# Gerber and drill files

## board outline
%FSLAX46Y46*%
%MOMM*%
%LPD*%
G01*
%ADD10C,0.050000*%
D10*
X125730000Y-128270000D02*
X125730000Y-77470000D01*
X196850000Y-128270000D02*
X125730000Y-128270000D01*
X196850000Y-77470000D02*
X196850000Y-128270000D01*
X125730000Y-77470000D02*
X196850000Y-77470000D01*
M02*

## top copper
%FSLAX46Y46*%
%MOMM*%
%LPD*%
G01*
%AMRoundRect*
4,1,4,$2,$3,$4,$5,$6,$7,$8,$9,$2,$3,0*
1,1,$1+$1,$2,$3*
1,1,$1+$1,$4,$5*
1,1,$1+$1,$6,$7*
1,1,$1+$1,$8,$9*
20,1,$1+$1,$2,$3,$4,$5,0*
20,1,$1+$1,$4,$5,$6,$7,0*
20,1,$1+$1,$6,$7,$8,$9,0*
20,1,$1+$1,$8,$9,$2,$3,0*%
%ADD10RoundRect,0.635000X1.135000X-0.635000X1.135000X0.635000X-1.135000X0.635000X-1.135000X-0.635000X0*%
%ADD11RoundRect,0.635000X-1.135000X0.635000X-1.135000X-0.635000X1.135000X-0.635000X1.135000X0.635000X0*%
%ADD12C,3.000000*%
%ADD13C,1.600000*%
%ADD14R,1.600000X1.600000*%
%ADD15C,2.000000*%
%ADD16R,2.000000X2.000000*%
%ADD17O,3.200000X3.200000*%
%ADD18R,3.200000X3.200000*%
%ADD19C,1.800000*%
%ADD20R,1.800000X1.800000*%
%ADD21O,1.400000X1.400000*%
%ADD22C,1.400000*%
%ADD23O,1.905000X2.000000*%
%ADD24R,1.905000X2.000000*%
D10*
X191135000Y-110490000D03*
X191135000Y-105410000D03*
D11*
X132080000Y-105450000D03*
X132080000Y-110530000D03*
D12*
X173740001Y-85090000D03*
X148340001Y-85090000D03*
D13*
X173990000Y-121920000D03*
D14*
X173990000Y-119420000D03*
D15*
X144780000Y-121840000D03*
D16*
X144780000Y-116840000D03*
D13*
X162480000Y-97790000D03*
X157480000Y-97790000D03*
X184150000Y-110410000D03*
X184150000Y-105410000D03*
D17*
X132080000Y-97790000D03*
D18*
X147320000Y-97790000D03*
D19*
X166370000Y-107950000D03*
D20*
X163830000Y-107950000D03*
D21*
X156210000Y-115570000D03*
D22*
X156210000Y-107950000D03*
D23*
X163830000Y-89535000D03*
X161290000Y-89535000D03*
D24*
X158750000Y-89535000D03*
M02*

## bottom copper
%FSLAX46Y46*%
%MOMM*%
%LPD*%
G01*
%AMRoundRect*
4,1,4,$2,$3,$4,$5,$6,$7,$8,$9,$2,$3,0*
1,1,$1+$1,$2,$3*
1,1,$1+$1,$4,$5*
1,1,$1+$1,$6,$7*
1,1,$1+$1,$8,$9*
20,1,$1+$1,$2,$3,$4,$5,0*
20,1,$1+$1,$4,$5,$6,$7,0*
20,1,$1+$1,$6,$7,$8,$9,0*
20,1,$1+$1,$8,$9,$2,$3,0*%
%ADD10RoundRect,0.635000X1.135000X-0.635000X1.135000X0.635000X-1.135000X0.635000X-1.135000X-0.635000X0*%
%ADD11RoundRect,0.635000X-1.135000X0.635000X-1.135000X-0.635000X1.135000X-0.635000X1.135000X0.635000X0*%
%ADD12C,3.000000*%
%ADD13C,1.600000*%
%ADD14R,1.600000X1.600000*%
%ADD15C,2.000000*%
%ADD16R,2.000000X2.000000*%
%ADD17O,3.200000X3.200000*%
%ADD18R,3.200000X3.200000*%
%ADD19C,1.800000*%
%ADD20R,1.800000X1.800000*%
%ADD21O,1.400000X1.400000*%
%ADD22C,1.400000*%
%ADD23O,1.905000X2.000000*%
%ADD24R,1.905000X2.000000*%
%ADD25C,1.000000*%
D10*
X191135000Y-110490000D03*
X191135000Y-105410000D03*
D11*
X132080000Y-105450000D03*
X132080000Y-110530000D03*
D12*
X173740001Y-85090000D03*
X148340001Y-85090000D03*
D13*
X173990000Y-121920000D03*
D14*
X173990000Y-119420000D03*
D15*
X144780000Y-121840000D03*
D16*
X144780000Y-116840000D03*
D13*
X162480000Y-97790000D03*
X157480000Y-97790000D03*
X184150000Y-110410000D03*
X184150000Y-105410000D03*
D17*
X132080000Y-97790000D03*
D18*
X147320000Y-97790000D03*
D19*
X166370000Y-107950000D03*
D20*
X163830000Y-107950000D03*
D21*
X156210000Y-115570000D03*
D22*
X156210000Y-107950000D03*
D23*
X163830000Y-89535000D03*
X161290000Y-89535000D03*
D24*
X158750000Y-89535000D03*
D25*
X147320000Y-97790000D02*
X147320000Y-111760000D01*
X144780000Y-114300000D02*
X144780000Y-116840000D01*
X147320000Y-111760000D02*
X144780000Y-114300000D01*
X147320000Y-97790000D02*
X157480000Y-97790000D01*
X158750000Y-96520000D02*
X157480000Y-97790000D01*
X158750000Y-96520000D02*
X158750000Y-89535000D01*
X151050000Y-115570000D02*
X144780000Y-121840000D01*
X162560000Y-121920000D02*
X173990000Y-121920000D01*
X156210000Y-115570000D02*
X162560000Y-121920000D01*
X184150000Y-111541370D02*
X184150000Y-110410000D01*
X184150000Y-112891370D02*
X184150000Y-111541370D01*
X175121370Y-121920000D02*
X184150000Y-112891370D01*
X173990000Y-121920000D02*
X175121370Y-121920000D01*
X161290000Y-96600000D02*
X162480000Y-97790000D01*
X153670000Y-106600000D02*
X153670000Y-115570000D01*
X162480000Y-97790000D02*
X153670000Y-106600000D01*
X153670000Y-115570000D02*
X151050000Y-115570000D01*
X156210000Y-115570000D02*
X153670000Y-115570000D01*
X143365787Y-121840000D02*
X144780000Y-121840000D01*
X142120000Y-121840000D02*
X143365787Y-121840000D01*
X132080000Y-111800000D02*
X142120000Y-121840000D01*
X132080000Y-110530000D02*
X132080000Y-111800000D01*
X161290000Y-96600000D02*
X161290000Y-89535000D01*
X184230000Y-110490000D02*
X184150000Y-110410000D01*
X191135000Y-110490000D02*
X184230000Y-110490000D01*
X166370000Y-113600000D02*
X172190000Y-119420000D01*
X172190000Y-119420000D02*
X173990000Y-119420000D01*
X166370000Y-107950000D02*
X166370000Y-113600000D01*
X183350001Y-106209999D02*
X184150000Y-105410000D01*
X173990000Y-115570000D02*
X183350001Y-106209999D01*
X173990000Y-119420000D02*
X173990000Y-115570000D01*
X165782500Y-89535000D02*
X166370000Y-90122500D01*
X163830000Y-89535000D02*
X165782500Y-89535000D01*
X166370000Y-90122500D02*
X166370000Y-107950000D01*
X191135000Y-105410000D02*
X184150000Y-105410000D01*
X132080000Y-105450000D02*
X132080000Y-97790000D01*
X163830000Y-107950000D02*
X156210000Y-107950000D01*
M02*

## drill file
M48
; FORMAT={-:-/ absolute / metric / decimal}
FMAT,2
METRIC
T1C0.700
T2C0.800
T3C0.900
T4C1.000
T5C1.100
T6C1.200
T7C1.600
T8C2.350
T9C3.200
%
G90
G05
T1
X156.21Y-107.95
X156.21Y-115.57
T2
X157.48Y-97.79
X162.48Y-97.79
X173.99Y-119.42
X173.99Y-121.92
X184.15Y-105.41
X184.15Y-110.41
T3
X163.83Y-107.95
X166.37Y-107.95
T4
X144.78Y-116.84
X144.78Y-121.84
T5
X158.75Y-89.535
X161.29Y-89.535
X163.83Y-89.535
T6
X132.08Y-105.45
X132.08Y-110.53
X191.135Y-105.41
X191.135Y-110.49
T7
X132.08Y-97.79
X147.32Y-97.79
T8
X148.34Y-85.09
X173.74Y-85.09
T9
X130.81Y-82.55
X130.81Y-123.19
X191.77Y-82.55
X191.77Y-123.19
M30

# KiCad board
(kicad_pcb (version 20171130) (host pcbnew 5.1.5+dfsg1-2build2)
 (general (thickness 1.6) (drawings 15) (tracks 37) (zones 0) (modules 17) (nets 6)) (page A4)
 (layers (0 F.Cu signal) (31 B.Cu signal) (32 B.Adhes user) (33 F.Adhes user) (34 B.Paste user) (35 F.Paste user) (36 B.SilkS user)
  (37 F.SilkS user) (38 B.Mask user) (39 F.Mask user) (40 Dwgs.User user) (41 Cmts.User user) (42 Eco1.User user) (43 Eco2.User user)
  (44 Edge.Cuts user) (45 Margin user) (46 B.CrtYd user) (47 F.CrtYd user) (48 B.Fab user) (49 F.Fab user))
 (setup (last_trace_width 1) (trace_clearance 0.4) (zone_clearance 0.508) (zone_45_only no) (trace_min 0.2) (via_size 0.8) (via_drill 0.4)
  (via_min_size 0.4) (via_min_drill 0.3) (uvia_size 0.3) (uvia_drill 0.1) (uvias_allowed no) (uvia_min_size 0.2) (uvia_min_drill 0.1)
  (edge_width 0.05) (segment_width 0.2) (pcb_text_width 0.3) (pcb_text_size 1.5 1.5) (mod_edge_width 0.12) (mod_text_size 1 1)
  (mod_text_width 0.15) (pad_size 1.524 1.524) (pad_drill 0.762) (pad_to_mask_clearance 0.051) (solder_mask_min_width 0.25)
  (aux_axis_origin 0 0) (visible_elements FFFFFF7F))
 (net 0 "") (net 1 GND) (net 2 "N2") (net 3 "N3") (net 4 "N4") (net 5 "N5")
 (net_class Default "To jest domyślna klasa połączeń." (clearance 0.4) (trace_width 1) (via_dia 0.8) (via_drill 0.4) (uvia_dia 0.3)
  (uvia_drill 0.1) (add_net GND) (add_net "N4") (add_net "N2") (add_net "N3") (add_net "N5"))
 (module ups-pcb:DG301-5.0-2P (layer F.Cu) (at 191.135 107.99 90)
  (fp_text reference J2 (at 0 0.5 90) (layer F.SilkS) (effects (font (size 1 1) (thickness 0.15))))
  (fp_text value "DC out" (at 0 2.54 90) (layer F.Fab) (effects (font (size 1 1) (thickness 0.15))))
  (pad 1 thru_hole roundrect (at -2.5 0 90) (size 2.54 3.54) (drill 1.2) (layers *.Cu *.Mask) (roundrect_rratio 0.25) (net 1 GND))
  (pad 2 thru_hole roundrect (at 2.58 0 90) (size 2.54 3.54) (drill 1.2) (layers *.Cu *.Mask) (roundrect_rratio 0.25) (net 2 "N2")))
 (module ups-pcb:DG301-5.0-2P (layer F.Cu) (at 132.08 107.95 270)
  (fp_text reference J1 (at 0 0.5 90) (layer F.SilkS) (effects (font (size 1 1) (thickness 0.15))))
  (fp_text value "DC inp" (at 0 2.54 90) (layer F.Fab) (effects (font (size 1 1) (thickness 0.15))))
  (pad 1 thru_hole roundrect (at -2.5 0 270) (size 2.54 3.54) (drill 1.2) (layers *.Cu *.Mask) (roundrect_rratio 0.25) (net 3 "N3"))
  (pad 2 thru_hole roundrect (at 2.58 0 270) (size 2.54 3.54) (drill 1.2) (layers *.Cu *.Mask) (roundrect_rratio 0.25) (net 1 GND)))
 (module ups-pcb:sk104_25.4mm (layer F.Cu) (at 161.040001 85.09)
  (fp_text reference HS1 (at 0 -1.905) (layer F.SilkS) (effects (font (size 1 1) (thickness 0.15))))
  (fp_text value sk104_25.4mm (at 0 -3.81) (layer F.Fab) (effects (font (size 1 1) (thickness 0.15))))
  (pad "" np_thru_hole circle (at 12.7 0) (size 3 3) (drill 2.35) (layers *.Cu *.Mask))
  (pad "" np_thru_hole circle (at -12.7 0) (size 3 3) (drill 2.35) (layers *.Cu *.Mask)))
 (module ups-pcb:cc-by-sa (layer F.Cu) (at 159.385 121.92)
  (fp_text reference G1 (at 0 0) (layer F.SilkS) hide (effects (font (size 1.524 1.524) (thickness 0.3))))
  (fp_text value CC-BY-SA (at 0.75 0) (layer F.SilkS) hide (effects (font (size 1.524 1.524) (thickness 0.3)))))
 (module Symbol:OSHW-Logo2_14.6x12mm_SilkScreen (layer F.Cu) (at 186.055 93.98)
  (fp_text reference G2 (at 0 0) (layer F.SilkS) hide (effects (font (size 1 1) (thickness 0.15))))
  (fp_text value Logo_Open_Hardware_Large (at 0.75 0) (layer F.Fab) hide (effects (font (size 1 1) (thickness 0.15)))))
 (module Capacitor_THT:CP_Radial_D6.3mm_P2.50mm (layer F.Cu) (at 173.99 119.42 270)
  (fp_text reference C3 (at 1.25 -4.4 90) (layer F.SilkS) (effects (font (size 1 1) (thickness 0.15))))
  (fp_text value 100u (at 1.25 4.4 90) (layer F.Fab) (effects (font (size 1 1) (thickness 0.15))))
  (pad 2 thru_hole circle (at 2.5 0 270) (size 1.6 1.6) (drill 0.8) (layers *.Cu *.Mask) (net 1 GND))
  (pad 1 thru_hole rect (at 0 0 270) (size 1.6 1.6) (drill 0.8) (layers *.Cu *.Mask) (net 2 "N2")))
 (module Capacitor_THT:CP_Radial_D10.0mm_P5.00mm (layer F.Cu) (at 144.78 116.84 270)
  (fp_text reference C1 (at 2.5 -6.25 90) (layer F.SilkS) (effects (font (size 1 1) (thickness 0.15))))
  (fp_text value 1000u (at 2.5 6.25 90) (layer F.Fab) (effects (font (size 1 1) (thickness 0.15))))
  (pad 2 thru_hole circle (at 5 0 270) (size 2 2) (drill 1) (layers *.Cu *.Mask) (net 1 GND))
  (pad 1 thru_hole rect (at 0 0 270) (size 2 2) (drill 1) (layers *.Cu *.Mask) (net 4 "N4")))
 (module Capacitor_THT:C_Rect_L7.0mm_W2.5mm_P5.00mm (layer F.Cu) (at 157.48 97.79)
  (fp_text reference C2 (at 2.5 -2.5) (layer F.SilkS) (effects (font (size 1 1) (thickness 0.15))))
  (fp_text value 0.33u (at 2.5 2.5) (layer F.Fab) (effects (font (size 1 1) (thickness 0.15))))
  (pad 2 thru_hole circle (at 5 0) (size 1.6 1.6) (drill 0.8) (layers *.Cu *.Mask) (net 1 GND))
  (pad 1 thru_hole circle (at 0 0) (size 1.6 1.6) (drill 0.8) (layers *.Cu *.Mask) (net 4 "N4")))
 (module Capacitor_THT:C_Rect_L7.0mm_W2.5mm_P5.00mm (layer F.Cu) (at 184.15 105.41 270)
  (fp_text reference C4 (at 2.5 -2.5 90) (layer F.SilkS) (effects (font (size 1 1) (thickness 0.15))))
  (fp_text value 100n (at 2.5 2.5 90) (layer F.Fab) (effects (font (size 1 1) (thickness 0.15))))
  (pad 2 thru_hole circle (at 5 0 270) (size 1.6 1.6) (drill 0.8) (layers *.Cu *.Mask) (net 1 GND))
  (pad 1 thru_hole circle (at 0 0 270) (size 1.6 1.6) (drill 0.8) (layers *.Cu *.Mask) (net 2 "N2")))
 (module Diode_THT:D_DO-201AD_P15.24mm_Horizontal (layer F.Cu) (at 147.32 97.79 180)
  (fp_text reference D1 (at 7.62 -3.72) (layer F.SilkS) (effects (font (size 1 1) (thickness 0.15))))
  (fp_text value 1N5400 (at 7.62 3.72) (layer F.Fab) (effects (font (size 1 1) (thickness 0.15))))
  (pad 2 thru_hole oval (at 15.24 0 180) (size 3.2 3.2) (drill 1.6) (layers *.Cu *.Mask) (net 3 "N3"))
  (pad 1 thru_hole rect (at 0 0 180) (size 3.2 3.2) (drill 1.6) (layers *.Cu *.Mask) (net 4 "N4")))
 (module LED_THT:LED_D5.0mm (layer F.Cu) (at 163.83 107.95)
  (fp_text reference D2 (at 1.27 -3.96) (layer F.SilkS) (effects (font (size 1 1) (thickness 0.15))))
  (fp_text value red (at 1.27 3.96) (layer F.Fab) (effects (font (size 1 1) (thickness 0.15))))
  (pad 2 thru_hole circle (at 2.54 0) (size 1.8 1.8) (drill 0.9) (layers *.Cu *.Mask) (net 2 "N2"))
  (pad 1 thru_hole rect (at 0 0) (size 1.8 1.8) (drill 0.9) (layers *.Cu *.Mask) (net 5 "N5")))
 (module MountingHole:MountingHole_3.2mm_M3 (layer F.Cu) (at 130.81 82.55)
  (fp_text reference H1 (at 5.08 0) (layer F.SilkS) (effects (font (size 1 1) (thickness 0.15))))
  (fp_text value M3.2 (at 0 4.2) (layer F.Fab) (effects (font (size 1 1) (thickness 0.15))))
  (pad 1 np_thru_hole circle (at 0 0) (size 3.2 3.2) (drill 3.2) (layers *.Cu *.Mask)))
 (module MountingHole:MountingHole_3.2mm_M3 (layer F.Cu) (at 191.77 82.55)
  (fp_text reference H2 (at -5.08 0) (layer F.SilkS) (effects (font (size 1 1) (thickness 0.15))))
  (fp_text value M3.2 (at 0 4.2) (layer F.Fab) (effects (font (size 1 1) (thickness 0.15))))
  (pad 1 np_thru_hole circle (at 0 0) (size 3.2 3.2) (drill 3.2) (layers *.Cu *.Mask)))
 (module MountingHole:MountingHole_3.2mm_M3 (layer F.Cu) (at 191.77 123.19)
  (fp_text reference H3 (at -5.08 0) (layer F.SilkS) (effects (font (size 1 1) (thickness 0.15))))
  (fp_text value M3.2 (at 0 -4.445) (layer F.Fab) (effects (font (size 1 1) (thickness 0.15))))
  (pad 1 np_thru_hole circle (at 0 0) (size 3.2 3.2) (drill 3.2) (layers *.Cu *.Mask)))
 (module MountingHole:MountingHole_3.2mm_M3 (layer F.Cu) (at 130.81 123.19)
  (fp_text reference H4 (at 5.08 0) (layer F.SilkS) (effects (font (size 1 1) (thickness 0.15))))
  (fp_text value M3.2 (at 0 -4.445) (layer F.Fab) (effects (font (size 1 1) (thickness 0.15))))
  (pad 1 np_thru_hole circle (at 0 0) (size 3.2 3.2) (drill 3.2) (layers *.Cu *.Mask)))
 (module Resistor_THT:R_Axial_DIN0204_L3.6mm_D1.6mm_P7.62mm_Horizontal (layer F.Cu) (at 156.21 107.95 270)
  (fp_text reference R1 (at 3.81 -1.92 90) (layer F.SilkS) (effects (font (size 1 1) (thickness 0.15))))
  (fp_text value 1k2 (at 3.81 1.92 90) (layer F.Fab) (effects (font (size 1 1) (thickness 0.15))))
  (pad 2 thru_hole oval (at 7.62 0 270) (size 1.4 1.4) (drill 0.7) (layers *.Cu *.Mask) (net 1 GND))
  (pad 1 thru_hole circle (at 0 0 270) (size 1.4 1.4) (drill 0.7) (layers *.Cu *.Mask) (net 5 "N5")))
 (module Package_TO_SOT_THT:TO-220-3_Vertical (layer F.Cu) (at 158.75 89.535)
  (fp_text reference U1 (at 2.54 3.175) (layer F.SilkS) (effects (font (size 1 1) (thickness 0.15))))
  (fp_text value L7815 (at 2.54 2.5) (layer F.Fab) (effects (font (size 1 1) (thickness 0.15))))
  (pad 3 thru_hole oval (at 5.08 0) (size 1.905 2) (drill 1.1) (layers *.Cu *.Mask) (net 2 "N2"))
  (pad 2 thru_hole oval (at 2.54 0) (size 1.905 2) (drill 1.1) (layers *.Cu *.Mask) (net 1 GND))
  (pad 1 thru_hole rect (at 0 0) (size 1.905 2) (drill 1.1) (layers *.Cu *.Mask) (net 4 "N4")))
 (gr_line (start 125.73 128.27) (end 125.73 77.47) (layer Edge.Cuts) (width 0.05))
 (gr_line (start 196.85 128.27) (end 125.73 128.27) (layer Edge.Cuts) (width 0.05))
 (gr_line (start 196.85 77.47) (end 196.85 128.27) (layer Edge.Cuts) (width 0.05))
 (gr_line (start 125.73 77.47) (end 196.85 77.47) (layer Edge.Cuts) (width 0.05))
 (segment (start 147.32 97.79) (end 147.32 111.76) (width 1) (layer B.Cu) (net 4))
 (segment (start 144.78 114.3) (end 144.78 116.84) (width 1) (layer B.Cu) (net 4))
 (segment (start 147.32 111.76) (end 144.78 114.3) (width 1) (layer B.Cu) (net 4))
 (segment (start 147.32 97.79) (end 157.48 97.79) (width 1) (layer B.Cu) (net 4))
 (segment (start 158.75 96.52) (end 157.48 97.79) (width 1) (layer B.Cu) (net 4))
 (segment (start 158.75 96.52) (end 158.75 89.535) (width 1) (layer B.Cu) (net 4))
 (segment (start 151.05 115.57) (end 144.78 121.84) (width 1) (layer B.Cu) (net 1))
 (segment (start 162.56 121.92) (end 173.99 121.92) (width 1) (layer B.Cu) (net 1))
 (segment (start 156.21 115.57) (end 162.56 121.92) (width 1) (layer B.Cu) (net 1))
 (segment (start 184.15 111.54137) (end 184.15 110.41) (width 1) (layer B.Cu) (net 1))
 (segment (start 184.15 112.89137) (end 184.15 111.54137) (width 1) (layer B.Cu) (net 1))
 (segment (start 175.12137 121.92) (end 184.15 112.89137) (width 1) (layer B.Cu) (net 1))
 (segment (start 173.99 121.92) (end 175.12137 121.92) (width 1) (layer B.Cu) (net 1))
 (segment (start 161.29 96.6) (end 162.48 97.79) (width 1) (layer B.Cu) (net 1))
 (segment (start 153.67 106.6) (end 153.67 115.57) (width 1) (layer B.Cu) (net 1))
 (segment (start 162.48 97.79) (end 153.67 106.6) (width 1) (layer B.Cu) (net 1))
 (segment (start 153.67 115.57) (end 151.05 115.57) (width 1) (layer B.Cu) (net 1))
 (segment (start 156.21 115.57) (end 153.67 115.57) (width 1) (layer B.Cu) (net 1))
 (segment (start 143.365787 121.84) (end 144.78 121.84) (width 1) (layer B.Cu) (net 1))
 (segment (start 142.12 121.84) (end 143.365787 121.84) (width 1) (layer B.Cu) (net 1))
 (segment (start 132.08 111.8) (end 142.12 121.84) (width 1) (layer B.Cu) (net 1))
 (segment (start 132.08 110.53) (end 132.08 111.8) (width 1) (layer B.Cu) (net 1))
 (segment (start 161.29 96.6) (end 161.29 89.535) (width 1) (layer B.Cu) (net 1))
 (segment (start 184.23 110.49) (end 184.15 110.41) (width 1) (layer B.Cu) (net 1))
 (segment (start 191.135 110.49) (end 184.23 110.49) (width 1) (layer B.Cu) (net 1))
 (segment (start 166.37 113.6) (end 172.19 119.42) (width 1) (layer B.Cu) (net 2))
 (segment (start 172.19 119.42) (end 173.99 119.42) (width 1) (layer B.Cu) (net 2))
 (segment (start 166.37 107.95) (end 166.37 113.6) (width 1) (layer B.Cu) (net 2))
 (segment (start 183.350001 106.209999) (end 184.15 105.41) (width 1) (layer B.Cu) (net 2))
 (segment (start 173.99 115.57) (end 183.350001 106.209999) (width 1) (layer B.Cu) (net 2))
 (segment (start 173.99 119.42) (end 173.99 115.57) (width 1) (layer B.Cu) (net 2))
 (segment (start 165.7825 89.535) (end 166.37 90.1225) (width 1) (layer B.Cu) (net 2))
 (segment (start 163.83 89.535) (end 165.7825 89.535) (width 1) (layer B.Cu) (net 2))
 (segment (start 166.37 90.1225) (end 166.37 107.95) (width 1) (layer B.Cu) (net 2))
 (segment (start 191.135 105.41) (end 184.15 105.41) (width 1) (layer B.Cu) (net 2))
 (segment (start 132.08 105.45) (end 132.08 97.79) (width 1) (layer B.Cu) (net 3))
 (segment (start 163.83 107.95) (end 156.21 107.95) (width 1) (layer B.Cu) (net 5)))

